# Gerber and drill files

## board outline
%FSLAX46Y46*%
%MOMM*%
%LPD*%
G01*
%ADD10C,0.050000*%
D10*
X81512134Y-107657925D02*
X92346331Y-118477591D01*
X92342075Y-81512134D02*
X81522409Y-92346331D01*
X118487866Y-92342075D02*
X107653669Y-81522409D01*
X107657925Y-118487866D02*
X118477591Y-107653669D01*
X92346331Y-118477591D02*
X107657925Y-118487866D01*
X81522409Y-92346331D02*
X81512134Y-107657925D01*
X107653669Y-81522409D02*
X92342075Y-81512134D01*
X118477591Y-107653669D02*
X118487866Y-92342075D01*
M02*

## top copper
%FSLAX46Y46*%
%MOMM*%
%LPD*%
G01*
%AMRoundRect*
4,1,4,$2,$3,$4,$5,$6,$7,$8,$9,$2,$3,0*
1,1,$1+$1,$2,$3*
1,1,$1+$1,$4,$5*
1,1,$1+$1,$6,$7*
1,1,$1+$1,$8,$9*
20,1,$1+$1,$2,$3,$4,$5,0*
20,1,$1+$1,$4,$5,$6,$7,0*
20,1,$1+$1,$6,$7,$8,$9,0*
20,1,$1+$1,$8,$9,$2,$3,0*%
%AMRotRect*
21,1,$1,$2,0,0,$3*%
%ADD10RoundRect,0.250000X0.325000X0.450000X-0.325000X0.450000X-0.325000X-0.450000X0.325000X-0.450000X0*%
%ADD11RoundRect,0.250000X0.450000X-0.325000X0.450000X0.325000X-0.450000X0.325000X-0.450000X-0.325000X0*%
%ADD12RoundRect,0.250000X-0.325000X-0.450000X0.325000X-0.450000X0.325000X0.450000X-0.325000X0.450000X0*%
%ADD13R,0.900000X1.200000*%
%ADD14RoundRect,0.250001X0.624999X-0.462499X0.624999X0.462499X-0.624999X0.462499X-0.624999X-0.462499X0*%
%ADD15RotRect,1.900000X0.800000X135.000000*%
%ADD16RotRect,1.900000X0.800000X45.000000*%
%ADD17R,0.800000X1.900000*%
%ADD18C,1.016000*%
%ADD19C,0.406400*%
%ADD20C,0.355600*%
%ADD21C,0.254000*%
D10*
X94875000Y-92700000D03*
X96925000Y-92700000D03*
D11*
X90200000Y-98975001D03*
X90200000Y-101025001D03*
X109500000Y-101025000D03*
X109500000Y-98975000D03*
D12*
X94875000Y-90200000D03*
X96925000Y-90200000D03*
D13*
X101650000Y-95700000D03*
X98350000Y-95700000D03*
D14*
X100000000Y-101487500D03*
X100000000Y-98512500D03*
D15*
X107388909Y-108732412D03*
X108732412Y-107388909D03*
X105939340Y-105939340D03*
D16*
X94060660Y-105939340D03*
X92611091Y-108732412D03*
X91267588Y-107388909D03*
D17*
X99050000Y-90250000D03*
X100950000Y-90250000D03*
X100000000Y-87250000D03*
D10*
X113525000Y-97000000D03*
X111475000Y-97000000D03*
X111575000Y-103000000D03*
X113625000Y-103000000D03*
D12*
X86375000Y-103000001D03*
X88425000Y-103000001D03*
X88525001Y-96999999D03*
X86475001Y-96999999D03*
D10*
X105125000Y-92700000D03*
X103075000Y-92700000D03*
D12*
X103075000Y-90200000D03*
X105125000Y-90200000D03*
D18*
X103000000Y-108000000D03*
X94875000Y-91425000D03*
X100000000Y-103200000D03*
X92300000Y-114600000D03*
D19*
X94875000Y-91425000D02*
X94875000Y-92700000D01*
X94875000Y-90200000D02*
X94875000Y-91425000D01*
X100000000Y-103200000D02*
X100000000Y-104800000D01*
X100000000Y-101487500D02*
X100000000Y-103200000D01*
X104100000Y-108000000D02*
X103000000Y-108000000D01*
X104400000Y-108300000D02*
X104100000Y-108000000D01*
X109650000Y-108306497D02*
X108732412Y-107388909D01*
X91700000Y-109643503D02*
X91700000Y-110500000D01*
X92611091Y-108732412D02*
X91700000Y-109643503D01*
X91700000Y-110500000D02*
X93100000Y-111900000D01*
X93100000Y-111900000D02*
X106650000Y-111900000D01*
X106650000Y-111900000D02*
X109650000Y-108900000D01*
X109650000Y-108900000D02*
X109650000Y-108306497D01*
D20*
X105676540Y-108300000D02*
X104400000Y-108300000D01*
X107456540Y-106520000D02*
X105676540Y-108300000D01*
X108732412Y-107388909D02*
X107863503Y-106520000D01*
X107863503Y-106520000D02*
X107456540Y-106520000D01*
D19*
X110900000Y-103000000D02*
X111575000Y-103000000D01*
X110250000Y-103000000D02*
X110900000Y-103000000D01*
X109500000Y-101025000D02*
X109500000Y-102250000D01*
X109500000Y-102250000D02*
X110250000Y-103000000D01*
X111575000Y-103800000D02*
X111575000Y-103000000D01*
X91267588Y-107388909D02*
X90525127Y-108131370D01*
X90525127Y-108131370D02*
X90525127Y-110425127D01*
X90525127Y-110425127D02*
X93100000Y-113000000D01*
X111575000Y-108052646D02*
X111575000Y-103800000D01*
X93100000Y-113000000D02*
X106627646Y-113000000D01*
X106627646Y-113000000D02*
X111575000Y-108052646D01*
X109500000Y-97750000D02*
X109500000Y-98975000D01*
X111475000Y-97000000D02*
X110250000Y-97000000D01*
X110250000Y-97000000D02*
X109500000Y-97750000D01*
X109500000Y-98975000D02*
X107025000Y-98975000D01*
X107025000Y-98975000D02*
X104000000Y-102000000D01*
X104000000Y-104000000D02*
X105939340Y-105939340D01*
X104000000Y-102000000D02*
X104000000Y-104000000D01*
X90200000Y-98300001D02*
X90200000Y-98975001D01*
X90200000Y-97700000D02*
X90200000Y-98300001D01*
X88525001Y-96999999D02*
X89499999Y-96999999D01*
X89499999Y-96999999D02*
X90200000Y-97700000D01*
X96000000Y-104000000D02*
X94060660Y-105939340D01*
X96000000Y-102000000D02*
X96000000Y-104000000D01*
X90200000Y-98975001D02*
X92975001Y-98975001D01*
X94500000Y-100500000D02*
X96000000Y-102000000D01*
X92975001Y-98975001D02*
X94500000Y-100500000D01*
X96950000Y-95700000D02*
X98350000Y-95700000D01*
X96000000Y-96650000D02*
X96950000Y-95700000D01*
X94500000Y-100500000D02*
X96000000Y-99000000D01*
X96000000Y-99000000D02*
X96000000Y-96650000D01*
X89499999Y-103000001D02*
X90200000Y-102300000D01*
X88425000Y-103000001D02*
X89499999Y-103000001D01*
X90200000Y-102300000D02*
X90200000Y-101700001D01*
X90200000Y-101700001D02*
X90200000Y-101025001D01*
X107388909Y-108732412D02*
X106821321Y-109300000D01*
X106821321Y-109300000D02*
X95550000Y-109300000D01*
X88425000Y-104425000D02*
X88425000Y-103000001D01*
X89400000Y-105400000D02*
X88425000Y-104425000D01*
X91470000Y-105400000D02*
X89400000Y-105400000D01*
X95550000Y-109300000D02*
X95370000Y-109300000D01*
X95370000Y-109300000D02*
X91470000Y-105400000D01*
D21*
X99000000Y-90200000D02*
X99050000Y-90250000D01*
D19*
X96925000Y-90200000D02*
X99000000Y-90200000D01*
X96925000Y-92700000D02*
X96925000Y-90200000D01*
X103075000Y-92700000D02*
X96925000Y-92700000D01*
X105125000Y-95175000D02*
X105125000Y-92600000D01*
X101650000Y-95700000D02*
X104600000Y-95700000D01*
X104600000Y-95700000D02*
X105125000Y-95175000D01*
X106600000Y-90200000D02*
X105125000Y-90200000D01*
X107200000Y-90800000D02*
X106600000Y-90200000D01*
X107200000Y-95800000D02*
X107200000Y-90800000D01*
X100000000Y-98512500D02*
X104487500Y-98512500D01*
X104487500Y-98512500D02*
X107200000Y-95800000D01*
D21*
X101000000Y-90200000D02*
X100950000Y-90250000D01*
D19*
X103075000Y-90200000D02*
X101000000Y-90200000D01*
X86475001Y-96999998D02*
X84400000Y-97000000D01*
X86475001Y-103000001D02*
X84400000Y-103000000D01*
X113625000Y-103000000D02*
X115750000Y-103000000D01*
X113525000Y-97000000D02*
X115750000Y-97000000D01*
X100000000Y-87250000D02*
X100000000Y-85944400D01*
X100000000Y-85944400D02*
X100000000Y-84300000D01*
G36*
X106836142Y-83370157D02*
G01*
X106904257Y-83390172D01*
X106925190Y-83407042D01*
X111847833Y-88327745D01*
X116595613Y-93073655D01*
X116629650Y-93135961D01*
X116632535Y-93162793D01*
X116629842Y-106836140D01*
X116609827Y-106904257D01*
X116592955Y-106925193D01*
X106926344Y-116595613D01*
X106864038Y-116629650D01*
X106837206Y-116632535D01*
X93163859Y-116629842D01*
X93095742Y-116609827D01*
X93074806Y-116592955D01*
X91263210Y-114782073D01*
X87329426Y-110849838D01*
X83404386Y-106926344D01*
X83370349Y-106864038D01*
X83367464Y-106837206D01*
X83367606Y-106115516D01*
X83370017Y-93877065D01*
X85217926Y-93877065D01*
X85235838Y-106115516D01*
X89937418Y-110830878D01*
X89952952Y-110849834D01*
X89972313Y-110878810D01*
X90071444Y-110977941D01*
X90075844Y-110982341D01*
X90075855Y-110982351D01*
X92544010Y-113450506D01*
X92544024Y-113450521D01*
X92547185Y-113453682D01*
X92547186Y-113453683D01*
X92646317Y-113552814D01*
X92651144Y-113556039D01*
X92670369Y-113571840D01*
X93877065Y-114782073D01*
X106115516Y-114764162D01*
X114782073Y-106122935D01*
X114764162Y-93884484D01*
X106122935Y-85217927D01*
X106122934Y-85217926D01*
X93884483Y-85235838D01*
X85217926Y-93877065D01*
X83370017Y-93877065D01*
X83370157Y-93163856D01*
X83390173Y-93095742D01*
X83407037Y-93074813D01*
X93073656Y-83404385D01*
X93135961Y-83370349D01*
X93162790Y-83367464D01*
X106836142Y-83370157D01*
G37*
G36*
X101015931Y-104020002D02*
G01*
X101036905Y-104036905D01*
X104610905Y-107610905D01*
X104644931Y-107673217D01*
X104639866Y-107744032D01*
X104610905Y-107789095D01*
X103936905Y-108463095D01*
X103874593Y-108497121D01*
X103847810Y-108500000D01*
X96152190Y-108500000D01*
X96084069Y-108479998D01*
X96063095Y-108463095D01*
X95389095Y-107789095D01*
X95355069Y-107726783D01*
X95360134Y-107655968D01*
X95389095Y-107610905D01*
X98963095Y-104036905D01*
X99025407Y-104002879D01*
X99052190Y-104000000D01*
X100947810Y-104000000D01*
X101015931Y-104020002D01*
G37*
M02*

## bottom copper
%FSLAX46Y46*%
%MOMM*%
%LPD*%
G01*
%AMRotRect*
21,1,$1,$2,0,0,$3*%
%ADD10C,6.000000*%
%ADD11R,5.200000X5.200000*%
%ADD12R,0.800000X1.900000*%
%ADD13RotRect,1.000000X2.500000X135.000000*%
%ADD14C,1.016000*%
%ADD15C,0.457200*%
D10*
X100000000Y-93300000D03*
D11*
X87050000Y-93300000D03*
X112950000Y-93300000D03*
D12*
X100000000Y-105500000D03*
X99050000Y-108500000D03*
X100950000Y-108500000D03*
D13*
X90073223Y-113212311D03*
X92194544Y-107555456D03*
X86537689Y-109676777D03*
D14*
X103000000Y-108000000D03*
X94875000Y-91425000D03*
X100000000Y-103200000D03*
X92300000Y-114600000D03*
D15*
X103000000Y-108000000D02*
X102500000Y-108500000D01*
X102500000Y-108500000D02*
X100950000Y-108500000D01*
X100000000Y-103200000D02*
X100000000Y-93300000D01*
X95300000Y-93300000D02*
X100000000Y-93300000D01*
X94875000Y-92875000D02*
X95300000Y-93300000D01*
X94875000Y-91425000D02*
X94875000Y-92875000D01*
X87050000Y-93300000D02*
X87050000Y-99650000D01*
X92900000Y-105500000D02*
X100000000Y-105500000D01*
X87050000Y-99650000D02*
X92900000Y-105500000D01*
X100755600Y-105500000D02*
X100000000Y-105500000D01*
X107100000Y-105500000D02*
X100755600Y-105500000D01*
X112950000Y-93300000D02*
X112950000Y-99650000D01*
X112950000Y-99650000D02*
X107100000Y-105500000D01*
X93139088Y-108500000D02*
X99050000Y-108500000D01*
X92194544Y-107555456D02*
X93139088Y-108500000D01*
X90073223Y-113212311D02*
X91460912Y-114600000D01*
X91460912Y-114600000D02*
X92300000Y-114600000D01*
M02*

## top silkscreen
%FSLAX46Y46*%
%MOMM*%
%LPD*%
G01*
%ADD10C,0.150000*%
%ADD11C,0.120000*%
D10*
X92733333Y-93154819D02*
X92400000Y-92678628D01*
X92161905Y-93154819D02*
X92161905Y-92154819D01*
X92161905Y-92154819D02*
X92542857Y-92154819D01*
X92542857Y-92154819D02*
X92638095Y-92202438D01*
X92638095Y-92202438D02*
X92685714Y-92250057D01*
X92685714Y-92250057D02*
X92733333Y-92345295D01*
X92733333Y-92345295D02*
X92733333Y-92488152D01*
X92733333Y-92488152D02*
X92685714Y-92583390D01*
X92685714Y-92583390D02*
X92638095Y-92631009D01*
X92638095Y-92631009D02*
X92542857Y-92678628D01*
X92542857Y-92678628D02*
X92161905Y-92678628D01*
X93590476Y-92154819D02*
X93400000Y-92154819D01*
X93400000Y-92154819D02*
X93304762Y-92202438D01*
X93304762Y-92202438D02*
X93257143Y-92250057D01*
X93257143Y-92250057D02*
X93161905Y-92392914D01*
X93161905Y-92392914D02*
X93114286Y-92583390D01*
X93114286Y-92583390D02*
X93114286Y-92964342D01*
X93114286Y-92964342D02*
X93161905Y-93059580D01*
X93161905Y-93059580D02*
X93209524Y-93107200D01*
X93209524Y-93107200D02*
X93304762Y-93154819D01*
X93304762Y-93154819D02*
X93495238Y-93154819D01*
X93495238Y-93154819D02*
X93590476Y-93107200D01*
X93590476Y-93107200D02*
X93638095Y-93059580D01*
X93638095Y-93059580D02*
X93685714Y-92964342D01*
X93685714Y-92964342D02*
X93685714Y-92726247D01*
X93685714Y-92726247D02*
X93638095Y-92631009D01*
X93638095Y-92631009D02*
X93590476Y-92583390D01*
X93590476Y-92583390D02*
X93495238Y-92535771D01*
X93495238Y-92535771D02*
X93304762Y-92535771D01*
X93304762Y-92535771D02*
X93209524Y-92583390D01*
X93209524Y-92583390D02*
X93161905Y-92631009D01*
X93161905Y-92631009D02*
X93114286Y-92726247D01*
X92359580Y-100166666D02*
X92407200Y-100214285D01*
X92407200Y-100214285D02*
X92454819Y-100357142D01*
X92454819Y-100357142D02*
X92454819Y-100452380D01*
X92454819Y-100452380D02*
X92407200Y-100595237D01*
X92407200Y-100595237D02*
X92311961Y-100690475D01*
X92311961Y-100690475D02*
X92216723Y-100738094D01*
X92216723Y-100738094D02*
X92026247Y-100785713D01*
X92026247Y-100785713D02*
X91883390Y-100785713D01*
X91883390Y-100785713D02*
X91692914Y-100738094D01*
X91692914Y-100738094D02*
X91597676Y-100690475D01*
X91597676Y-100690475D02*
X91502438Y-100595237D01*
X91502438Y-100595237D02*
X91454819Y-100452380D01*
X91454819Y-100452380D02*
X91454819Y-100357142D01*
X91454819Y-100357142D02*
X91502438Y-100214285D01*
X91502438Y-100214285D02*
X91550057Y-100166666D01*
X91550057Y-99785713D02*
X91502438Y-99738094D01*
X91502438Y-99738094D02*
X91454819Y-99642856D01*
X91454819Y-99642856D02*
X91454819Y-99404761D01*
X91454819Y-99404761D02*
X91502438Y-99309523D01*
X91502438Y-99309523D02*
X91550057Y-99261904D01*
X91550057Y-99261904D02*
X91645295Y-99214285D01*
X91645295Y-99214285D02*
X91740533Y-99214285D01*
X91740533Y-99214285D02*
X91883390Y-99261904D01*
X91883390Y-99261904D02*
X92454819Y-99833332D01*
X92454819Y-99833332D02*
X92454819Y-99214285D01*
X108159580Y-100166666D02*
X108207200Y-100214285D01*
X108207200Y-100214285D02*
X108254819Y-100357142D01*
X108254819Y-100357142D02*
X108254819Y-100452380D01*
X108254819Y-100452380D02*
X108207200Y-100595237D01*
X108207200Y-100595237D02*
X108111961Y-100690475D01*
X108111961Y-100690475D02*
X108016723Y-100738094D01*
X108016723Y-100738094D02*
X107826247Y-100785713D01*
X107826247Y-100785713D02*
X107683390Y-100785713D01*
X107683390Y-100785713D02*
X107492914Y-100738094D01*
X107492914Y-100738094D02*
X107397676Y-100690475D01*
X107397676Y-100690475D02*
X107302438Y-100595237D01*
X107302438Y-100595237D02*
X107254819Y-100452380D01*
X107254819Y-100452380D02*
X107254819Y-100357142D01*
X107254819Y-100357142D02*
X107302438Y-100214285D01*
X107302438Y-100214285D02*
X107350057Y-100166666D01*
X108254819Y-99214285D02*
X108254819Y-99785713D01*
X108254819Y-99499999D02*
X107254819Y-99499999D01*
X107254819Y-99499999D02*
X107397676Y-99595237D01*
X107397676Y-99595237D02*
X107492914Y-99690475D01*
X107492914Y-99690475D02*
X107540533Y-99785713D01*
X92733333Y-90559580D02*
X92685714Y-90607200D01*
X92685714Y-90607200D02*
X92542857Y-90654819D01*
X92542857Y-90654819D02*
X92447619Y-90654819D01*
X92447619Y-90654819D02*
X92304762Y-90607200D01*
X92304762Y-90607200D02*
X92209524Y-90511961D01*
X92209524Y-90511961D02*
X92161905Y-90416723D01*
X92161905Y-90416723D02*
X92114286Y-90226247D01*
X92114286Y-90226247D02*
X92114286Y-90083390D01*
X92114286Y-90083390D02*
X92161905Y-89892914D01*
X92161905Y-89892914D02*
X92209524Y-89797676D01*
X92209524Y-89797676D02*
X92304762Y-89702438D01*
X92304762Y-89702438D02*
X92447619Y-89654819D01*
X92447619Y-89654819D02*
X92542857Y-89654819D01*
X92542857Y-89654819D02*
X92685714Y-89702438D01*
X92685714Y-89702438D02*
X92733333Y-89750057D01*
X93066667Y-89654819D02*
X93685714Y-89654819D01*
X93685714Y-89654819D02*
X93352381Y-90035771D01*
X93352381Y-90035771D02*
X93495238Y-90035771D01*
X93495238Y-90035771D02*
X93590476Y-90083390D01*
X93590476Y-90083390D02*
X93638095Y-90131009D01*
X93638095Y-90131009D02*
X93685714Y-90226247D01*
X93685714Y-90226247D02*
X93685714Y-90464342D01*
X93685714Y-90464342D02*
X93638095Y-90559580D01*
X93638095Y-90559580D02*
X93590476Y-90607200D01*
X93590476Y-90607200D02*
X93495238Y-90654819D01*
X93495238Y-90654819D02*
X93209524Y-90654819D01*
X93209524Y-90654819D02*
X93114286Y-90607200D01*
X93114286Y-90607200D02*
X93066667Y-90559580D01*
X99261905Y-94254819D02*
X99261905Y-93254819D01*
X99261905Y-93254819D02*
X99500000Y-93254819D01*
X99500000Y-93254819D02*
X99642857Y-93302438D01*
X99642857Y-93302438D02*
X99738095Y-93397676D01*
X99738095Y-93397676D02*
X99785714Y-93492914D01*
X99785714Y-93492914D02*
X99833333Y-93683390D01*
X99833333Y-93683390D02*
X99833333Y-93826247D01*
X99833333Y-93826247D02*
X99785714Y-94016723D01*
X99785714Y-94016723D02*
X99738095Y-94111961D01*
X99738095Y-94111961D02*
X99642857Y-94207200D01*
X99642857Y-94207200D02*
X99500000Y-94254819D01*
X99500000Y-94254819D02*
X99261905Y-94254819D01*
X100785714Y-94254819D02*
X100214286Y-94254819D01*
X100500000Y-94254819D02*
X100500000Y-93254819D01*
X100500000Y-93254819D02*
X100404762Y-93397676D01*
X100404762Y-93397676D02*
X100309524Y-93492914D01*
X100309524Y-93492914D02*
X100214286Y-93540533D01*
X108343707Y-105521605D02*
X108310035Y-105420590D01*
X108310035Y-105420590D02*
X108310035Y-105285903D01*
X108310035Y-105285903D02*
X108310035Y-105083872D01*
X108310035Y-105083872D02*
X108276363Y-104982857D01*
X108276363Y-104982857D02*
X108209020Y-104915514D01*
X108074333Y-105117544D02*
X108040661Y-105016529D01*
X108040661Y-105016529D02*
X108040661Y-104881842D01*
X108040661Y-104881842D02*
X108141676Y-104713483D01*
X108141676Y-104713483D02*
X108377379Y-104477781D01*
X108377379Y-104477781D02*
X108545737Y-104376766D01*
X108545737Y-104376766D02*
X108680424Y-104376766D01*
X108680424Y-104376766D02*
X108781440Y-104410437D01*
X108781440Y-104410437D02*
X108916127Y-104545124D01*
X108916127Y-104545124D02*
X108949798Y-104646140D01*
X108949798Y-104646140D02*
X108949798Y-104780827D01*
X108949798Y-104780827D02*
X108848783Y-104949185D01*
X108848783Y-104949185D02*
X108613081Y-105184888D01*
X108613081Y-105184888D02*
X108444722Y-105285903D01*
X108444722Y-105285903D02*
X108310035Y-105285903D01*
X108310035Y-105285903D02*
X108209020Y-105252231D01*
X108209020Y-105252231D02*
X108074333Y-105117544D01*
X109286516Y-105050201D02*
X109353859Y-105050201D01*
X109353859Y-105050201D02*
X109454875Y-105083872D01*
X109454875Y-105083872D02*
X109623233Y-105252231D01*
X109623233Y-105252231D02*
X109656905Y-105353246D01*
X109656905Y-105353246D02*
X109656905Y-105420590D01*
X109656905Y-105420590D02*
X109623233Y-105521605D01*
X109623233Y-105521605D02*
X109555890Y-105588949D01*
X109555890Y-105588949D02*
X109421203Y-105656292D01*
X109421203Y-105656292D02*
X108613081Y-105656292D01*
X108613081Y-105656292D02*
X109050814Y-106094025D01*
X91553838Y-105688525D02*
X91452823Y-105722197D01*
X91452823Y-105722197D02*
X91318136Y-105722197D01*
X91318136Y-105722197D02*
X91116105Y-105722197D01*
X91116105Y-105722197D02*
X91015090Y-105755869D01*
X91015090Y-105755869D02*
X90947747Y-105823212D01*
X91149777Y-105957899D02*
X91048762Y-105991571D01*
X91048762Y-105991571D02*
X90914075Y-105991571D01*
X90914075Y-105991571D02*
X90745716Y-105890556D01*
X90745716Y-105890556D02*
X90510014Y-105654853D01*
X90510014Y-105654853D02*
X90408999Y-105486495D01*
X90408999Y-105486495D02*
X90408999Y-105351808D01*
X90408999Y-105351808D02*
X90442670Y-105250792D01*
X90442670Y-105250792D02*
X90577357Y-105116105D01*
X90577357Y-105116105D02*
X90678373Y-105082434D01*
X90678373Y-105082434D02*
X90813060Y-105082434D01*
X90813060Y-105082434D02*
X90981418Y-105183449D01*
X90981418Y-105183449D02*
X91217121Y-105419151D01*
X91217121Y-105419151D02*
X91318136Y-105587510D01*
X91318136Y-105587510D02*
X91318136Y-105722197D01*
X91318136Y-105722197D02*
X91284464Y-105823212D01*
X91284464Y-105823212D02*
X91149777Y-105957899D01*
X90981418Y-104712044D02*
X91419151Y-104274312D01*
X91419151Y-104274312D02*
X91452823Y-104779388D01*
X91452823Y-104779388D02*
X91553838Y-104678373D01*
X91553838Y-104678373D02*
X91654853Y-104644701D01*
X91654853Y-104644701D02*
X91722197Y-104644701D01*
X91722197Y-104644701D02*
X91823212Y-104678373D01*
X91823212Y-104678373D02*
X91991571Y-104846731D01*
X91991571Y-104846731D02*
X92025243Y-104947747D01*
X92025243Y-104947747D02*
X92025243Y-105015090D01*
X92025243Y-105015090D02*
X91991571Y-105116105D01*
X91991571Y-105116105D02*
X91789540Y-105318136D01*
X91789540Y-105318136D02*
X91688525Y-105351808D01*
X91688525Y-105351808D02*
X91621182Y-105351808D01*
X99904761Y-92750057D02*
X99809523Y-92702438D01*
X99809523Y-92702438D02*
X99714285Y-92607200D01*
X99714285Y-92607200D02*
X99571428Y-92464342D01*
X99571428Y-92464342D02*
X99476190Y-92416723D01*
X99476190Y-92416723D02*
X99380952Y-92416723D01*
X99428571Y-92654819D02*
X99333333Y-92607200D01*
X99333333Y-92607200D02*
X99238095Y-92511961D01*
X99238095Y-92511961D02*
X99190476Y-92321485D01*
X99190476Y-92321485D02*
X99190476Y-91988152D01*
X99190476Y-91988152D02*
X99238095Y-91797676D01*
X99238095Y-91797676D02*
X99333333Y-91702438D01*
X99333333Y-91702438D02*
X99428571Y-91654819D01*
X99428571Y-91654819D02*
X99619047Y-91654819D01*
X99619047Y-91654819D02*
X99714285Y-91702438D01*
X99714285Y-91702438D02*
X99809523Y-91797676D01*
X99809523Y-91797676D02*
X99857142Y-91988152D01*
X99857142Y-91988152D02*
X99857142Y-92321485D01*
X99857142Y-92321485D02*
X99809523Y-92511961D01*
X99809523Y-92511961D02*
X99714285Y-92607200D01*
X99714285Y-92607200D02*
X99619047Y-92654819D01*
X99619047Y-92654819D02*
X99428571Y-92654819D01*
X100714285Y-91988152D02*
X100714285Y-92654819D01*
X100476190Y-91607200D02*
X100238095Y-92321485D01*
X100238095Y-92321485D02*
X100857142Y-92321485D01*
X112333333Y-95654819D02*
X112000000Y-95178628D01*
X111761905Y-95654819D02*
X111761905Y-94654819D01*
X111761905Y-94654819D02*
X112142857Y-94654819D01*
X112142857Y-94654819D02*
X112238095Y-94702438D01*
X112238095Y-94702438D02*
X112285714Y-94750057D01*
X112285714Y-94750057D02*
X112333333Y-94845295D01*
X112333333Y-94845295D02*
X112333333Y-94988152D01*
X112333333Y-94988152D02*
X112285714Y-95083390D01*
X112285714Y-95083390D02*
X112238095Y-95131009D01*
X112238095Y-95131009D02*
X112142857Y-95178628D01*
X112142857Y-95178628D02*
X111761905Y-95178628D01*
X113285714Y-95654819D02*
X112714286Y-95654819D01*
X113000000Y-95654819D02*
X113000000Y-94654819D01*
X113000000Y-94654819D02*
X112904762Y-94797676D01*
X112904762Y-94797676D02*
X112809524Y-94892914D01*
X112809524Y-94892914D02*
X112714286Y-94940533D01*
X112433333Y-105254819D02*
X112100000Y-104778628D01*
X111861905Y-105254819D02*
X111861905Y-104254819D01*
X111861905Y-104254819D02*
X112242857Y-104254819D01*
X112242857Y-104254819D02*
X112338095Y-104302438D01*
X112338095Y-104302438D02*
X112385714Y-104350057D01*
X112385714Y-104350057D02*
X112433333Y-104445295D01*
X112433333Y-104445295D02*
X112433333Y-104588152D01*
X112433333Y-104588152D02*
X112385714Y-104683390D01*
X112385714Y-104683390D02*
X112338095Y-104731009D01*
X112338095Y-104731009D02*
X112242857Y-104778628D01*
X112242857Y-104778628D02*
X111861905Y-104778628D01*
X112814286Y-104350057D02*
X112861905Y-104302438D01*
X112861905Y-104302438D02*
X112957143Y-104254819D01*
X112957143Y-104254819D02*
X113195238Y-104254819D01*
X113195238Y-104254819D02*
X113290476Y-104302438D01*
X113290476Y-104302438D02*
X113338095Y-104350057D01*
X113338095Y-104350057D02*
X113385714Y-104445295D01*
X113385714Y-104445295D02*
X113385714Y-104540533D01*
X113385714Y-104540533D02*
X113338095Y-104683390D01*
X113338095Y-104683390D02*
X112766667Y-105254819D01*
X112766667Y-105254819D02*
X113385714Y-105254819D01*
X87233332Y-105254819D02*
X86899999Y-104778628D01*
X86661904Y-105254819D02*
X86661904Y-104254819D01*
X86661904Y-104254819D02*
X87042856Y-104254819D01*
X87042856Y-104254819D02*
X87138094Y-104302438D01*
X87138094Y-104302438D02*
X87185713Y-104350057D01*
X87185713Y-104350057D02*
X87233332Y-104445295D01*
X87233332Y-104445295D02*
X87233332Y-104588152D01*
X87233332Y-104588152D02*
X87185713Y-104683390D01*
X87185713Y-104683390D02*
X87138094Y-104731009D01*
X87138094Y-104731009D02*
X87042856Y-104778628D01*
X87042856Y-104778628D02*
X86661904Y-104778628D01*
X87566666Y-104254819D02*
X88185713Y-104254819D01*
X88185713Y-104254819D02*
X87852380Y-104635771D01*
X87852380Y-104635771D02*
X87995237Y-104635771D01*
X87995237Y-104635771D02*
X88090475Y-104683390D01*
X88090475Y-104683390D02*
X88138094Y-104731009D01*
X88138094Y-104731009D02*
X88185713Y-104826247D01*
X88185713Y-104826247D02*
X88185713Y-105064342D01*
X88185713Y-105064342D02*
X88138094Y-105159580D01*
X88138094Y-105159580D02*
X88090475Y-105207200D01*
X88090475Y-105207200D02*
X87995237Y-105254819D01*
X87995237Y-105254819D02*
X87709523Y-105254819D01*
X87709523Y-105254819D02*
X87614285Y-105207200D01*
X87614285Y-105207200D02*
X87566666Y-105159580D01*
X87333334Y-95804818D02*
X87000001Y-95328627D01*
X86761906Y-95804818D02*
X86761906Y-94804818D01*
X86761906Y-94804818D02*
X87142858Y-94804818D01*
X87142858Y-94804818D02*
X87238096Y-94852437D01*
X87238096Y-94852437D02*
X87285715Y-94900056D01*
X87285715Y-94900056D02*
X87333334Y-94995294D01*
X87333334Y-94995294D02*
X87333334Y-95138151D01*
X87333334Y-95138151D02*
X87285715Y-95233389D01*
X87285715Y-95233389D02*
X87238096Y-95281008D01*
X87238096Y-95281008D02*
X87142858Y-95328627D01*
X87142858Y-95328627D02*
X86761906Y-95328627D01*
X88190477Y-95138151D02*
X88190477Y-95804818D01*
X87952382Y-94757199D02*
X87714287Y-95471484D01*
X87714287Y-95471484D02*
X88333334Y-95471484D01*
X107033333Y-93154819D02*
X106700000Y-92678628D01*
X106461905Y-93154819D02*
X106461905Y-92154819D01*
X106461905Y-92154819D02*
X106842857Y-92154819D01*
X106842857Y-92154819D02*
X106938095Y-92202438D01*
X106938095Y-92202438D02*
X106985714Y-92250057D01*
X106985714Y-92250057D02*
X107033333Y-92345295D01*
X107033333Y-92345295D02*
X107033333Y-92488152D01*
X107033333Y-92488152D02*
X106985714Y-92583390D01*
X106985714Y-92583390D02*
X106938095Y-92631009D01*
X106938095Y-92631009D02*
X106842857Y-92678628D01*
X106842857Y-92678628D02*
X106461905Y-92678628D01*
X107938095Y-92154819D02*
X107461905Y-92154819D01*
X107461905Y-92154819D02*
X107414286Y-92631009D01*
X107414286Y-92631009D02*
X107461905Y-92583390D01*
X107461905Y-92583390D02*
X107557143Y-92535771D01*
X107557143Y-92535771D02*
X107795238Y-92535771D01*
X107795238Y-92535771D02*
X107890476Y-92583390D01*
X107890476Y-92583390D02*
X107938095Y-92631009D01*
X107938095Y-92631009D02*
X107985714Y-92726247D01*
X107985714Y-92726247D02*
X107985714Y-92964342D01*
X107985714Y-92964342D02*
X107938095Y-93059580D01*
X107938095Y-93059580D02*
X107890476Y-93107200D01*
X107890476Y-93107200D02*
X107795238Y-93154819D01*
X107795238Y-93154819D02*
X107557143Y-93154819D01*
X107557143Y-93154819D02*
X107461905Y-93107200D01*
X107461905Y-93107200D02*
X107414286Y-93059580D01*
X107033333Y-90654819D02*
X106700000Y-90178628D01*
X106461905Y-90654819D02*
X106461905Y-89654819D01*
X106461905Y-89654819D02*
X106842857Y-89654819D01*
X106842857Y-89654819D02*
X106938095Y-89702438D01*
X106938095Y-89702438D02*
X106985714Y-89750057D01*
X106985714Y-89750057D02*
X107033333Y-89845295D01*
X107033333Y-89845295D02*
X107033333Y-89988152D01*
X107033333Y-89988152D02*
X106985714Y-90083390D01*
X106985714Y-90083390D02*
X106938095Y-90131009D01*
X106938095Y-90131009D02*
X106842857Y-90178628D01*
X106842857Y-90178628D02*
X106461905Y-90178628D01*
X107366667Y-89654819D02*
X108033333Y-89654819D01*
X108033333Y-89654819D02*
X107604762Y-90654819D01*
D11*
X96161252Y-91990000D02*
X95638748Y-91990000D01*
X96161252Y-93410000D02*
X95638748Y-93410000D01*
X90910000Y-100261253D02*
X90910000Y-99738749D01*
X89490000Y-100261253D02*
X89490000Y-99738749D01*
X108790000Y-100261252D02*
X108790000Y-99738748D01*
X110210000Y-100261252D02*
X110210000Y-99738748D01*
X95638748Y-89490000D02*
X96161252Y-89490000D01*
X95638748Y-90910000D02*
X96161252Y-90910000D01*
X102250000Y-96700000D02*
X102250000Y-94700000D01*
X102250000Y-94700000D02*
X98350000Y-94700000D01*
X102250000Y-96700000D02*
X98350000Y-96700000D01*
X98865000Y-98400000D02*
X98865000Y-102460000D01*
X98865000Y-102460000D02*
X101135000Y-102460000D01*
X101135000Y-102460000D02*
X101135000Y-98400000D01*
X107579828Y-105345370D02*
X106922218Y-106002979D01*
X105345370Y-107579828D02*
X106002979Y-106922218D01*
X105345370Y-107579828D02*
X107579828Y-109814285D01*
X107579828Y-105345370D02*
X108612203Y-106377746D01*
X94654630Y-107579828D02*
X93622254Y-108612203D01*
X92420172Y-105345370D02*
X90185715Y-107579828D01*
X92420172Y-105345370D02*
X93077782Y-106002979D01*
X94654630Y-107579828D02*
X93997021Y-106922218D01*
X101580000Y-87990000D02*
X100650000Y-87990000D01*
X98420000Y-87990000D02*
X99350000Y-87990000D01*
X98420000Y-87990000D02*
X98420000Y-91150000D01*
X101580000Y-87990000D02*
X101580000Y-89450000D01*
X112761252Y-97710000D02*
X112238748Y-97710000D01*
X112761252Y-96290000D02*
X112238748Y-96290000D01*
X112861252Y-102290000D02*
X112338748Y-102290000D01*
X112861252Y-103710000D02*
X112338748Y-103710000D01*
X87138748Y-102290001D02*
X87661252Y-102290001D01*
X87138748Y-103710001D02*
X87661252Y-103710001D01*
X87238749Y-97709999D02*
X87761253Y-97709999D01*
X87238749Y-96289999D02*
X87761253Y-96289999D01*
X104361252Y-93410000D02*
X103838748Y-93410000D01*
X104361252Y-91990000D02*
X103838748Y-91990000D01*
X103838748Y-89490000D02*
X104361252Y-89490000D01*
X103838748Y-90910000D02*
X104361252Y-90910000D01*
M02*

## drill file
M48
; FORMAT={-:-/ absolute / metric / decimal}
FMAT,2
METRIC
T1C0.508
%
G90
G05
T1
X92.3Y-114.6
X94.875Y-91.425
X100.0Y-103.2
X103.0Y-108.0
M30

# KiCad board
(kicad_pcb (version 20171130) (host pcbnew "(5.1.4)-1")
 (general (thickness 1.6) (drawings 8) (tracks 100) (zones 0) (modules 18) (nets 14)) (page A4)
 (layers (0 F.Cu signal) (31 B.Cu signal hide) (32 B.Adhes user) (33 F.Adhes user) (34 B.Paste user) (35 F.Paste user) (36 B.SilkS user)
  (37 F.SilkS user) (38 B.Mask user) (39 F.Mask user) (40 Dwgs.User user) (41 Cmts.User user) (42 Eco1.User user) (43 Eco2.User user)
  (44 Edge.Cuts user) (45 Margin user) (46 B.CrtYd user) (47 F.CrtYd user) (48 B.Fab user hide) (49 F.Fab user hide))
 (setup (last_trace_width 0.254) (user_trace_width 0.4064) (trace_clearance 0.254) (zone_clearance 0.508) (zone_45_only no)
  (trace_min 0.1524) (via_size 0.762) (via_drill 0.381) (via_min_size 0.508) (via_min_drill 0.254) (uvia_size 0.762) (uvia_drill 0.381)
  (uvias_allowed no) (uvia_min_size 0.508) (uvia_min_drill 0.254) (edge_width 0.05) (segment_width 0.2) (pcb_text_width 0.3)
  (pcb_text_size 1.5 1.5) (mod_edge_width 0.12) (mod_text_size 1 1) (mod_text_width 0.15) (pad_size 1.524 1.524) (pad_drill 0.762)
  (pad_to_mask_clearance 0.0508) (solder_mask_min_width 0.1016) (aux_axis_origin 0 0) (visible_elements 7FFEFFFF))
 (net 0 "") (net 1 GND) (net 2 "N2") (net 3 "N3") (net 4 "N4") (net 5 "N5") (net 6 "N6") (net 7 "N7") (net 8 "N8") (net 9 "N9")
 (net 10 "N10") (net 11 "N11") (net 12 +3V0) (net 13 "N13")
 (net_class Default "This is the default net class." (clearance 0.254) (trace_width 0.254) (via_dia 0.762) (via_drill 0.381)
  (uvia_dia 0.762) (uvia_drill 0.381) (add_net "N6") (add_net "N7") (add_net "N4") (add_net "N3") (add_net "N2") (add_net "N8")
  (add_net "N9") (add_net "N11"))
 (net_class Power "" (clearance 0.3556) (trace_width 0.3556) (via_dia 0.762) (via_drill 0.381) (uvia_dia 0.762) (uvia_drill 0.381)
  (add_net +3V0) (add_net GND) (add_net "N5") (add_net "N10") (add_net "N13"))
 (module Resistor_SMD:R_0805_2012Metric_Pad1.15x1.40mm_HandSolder (layer F.Cu) (at 95.9 92.7 180)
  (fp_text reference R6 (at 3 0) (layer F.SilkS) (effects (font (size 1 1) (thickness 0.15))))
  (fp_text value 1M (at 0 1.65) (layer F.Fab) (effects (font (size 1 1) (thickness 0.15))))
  (fp_line (start -0.261252 0.71) (end 0.261252 0.71) (layer F.SilkS) (width 0.12))
  (fp_line (start -0.261252 -0.71) (end 0.261252 -0.71) (layer F.SilkS) (width 0.12))
  (pad 2 smd roundrect (at 1.025 0 180) (size 1.15 1.4) (layers F.Cu F.Paste F.Mask) (roundrect_rratio 0.217391) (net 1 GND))
  (pad 1 smd roundrect (at -1.025 0 180) (size 1.15 1.4) (layers F.Cu F.Paste F.Mask) (roundrect_rratio 0.217391) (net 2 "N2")))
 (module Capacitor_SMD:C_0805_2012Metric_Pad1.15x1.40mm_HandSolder (layer F.Cu) (at 90.2 100.000001 90)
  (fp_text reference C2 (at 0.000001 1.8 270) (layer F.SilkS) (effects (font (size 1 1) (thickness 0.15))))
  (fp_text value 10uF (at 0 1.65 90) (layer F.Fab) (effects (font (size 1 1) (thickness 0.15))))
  (fp_line (start -0.261252 0.71) (end 0.261252 0.71) (layer F.SilkS) (width 0.12))
  (fp_line (start -0.261252 -0.71) (end 0.261252 -0.71) (layer F.SilkS) (width 0.12))
  (pad 2 smd roundrect (at 1.025 0 90) (size 1.15 1.4) (layers F.Cu F.Paste F.Mask) (roundrect_rratio 0.217391) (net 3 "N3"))
  (pad 1 smd roundrect (at -1.025 0 90) (size 1.15 1.4) (layers F.Cu F.Paste F.Mask) (roundrect_rratio 0.217391) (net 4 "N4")))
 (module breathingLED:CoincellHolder (layer B.Cu) (at 100 93.3) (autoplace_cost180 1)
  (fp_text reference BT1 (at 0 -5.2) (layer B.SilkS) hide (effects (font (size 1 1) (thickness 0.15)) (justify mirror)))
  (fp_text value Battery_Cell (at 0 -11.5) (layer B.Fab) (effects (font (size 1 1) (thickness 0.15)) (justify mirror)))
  (pad 2 smd circle (at 0 0) (size 6 6) (layers B.Cu B.Paste B.Mask) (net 1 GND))
  (pad 1 smd rect (at -12.95 0) (size 5.2 5.2) (layers B.Cu B.Paste B.Mask) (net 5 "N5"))
  (pad 1 smd rect (at 12.95 0) (size 5.2 5.2) (layers B.Cu B.Paste B.Mask) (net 5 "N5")))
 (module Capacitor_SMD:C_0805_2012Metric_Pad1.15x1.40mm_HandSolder (layer F.Cu) (at 109.5 100 90)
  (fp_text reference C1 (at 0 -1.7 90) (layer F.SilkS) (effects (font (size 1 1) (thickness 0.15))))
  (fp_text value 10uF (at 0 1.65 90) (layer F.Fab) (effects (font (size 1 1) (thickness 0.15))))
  (fp_line (start -0.261252 -0.71) (end 0.261252 -0.71) (layer F.SilkS) (width 0.12))
  (fp_line (start -0.261252 0.71) (end 0.261252 0.71) (layer F.SilkS) (width 0.12))
  (pad 1 smd roundrect (at -1.025 0 90) (size 1.15 1.4) (layers F.Cu F.Paste F.Mask) (roundrect_rratio 0.217391) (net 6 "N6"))
  (pad 2 smd roundrect (at 1.025 0 90) (size 1.15 1.4) (layers F.Cu F.Paste F.Mask) (roundrect_rratio 0.217391) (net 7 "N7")))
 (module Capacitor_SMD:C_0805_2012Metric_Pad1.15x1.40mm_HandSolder (layer F.Cu) (at 95.9 90.2)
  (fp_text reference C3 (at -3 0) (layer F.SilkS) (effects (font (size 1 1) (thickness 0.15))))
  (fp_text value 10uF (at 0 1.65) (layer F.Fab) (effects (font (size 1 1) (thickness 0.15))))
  (fp_line (start -0.261252 -0.71) (end 0.261252 -0.71) (layer F.SilkS) (width 0.12))
  (fp_line (start -0.261252 0.71) (end 0.261252 0.71) (layer F.SilkS) (width 0.12))
  (pad 1 smd roundrect (at -1.025 0) (size 1.15 1.4) (layers F.Cu F.Paste F.Mask) (roundrect_rratio 0.217391) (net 1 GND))
  (pad 2 smd roundrect (at 1.025 0) (size 1.15 1.4) (layers F.Cu F.Paste F.Mask) (roundrect_rratio 0.217391) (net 2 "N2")))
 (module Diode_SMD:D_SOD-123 (layer F.Cu) (at 100 95.7 180)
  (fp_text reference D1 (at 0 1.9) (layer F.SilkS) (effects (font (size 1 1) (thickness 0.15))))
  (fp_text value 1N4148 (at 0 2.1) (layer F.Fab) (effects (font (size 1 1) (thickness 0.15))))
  (fp_line (start -2.25 -1) (end -2.25 1) (layer F.SilkS) (width 0.12))
  (fp_line (start -2.25 1) (end 1.65 1) (layer F.SilkS) (width 0.12))
  (fp_line (start -2.25 -1) (end 1.65 -1) (layer F.SilkS) (width 0.12))
  (pad 1 smd rect (at -1.65 0 180) (size 0.9 1.2) (layers F.Cu F.Paste F.Mask) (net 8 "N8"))
  (pad 2 smd rect (at 1.65 0 180) (size 0.9 1.2) (layers F.Cu F.Paste F.Mask) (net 3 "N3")))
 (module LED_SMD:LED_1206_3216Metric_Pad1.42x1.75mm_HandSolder (layer F.Cu) (at 100 100 90)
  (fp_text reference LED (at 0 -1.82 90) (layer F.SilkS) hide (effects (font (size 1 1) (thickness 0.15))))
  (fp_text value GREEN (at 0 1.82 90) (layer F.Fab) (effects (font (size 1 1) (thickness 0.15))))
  (fp_line (start 1.6 -1.135) (end -2.46 -1.135) (layer F.SilkS) (width 0.12))
  (fp_line (start -2.46 -1.135) (end -2.46 1.135) (layer F.SilkS) (width 0.12))
  (fp_line (start -2.46 1.135) (end 1.6 1.135) (layer F.SilkS) (width 0.12))
  (pad 1 smd roundrect (at -1.4875 0 90) (size 1.425 1.75) (layers F.Cu F.Paste F.Mask) (roundrect_rratio 0.175439) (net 1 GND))
  (pad 2 smd roundrect (at 1.4875 0 90) (size 1.425 1.75) (layers F.Cu F.Paste F.Mask) (roundrect_rratio 0.175439) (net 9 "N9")))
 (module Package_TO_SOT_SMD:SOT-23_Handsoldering (layer B.Cu) (at 100 107 90)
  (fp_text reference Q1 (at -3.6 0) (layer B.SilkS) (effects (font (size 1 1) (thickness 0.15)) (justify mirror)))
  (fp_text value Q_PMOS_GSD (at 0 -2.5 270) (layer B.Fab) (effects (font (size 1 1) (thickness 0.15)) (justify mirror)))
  (pad 3 smd rect (at 1.5 0 90) (size 1.9 0.8) (layers B.Cu B.Paste B.Mask) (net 5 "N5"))
  (pad 2 smd rect (at -1.5 -0.95 90) (size 1.9 0.8) (layers B.Cu B.Paste B.Mask) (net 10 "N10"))
  (pad 1 smd rect (at -1.5 0.95 90) (size 1.9 0.8) (layers B.Cu B.Paste B.Mask) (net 1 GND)))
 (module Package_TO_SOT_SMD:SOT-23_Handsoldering (layer F.Cu) (at 107 107 135)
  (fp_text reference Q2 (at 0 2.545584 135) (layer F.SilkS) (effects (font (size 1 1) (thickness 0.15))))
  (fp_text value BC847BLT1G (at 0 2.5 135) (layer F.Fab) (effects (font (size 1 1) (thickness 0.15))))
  (fp_line (start 0.76 1.58) (end 0.76 0.65) (layer F.SilkS) (width 0.12))
  (fp_line (start 0.76 -1.58) (end 0.76 -0.65) (layer F.SilkS) (width 0.12))
  (fp_line (start 0.76 -1.58) (end -2.4 -1.58) (layer F.SilkS) (width 0.12))
  (fp_line (start 0.76 1.58) (end -0.7 1.58) (layer F.SilkS) (width 0.12))
  (pad 1 smd rect (at -1.5 -0.95 135) (size 1.9 0.8) (layers F.Cu F.Paste F.Mask) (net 4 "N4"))
  (pad 2 smd rect (at -1.5 0.95 135) (size 1.9 0.8) (layers F.Cu F.Paste F.Mask) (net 1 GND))
  (pad 3 smd rect (at 1.5 0 135) (size 1.9 0.8) (layers F.Cu F.Paste F.Mask) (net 7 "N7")))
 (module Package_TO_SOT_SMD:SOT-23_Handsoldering (layer F.Cu) (at 93 107 45)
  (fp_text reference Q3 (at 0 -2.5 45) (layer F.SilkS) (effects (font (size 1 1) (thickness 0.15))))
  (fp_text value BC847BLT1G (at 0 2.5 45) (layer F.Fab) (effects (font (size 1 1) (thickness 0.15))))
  (fp_line (start 0.76 1.58) (end -0.7 1.58) (layer F.SilkS) (width 0.12))
  (fp_line (start 0.76 -1.58) (end -2.4 -1.58) (layer F.SilkS) (width 0.12))
  (fp_line (start 0.76 -1.58) (end 0.76 -0.65) (layer F.SilkS) (width 0.12))
  (fp_line (start 0.76 1.58) (end 0.76 0.65) (layer F.SilkS) (width 0.12))
  (pad 3 smd rect (at 1.5 0 45) (size 1.9 0.8) (layers F.Cu F.Paste F.Mask) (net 3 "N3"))
  (pad 2 smd rect (at -1.5 0.95 45) (size 1.9 0.8) (layers F.Cu F.Paste F.Mask) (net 1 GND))
  (pad 1 smd rect (at -1.5 -0.95 45) (size 1.9 0.8) (layers F.Cu F.Paste F.Mask) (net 6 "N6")))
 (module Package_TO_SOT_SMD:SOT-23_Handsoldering (layer F.Cu) (at 100 88.75 90)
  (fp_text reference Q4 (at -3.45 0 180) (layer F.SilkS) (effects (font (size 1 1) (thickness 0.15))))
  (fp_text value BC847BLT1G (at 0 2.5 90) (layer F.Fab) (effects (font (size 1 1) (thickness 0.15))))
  (fp_line (start 0.76 1.58) (end 0.76 0.65) (layer F.SilkS) (width 0.12))
  (fp_line (start 0.76 -1.58) (end 0.76 -0.65) (layer F.SilkS) (width 0.12))
  (fp_line (start 0.76 -1.58) (end -2.4 -1.58) (layer F.SilkS) (width 0.12))
  (fp_line (start 0.76 1.58) (end -0.7 1.58) (layer F.SilkS) (width 0.12))
  (pad 1 smd rect (at -1.5 -0.95 90) (size 1.9 0.8) (layers F.Cu F.Paste F.Mask) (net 2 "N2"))
  (pad 2 smd rect (at -1.5 0.95 90) (size 1.9 0.8) (layers F.Cu F.Paste F.Mask) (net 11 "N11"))
  (pad 3 smd rect (at 1.5 0 90) (size 1.9 0.8) (layers F.Cu F.Paste F.Mask) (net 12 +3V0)))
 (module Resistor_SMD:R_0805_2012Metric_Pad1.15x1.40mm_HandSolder (layer F.Cu) (at 112.5 97 180)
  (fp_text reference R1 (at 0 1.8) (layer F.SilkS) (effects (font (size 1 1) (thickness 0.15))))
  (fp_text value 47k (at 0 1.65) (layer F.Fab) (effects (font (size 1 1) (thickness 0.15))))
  (fp_line (start -0.261252 -0.71) (end 0.261252 -0.71) (layer F.SilkS) (width 0.12))
  (fp_line (start -0.261252 0.71) (end 0.261252 0.71) (layer F.SilkS) (width 0.12))
  (pad 1 smd roundrect (at -1.025 0 180) (size 1.15 1.4) (layers F.Cu F.Paste F.Mask) (roundrect_rratio 0.217391) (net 12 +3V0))
  (pad 2 smd roundrect (at 1.025 0 180) (size 1.15 1.4) (layers F.Cu F.Paste F.Mask) (roundrect_rratio 0.217391) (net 7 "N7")))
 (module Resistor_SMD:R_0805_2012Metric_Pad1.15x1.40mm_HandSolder (layer F.Cu) (at 112.6 103 180)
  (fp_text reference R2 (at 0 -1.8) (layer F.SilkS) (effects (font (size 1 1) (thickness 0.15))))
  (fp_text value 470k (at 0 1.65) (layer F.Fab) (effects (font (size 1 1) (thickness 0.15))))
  (fp_line (start -0.261252 0.71) (end 0.261252 0.71) (layer F.SilkS) (width 0.12))
  (fp_line (start -0.261252 -0.71) (end 0.261252 -0.71) (layer F.SilkS) (width 0.12))
  (pad 2 smd roundrect (at 1.025 0 180) (size 1.15 1.4) (layers F.Cu F.Paste F.Mask) (roundrect_rratio 0.217391) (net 6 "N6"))
  (pad 1 smd roundrect (at -1.025 0 180) (size 1.15 1.4) (layers F.Cu F.Paste F.Mask) (roundrect_rratio 0.217391) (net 12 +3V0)))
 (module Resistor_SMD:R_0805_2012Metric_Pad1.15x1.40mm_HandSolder (layer F.Cu) (at 87.4 103.000001)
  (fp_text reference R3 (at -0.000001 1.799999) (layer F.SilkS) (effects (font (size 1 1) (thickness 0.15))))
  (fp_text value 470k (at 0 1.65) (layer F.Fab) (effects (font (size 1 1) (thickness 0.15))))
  (fp_line (start -0.261252 -0.71) (end 0.261252 -0.71) (layer F.SilkS) (width 0.12))
  (fp_line (start -0.261252 0.71) (end 0.261252 0.71) (layer F.SilkS) (width 0.12))
  (pad 1 smd roundrect (at -1.025 0) (size 1.15 1.4) (layers F.Cu F.Paste F.Mask) (roundrect_rratio 0.217391) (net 12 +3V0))
  (pad 2 smd roundrect (at 1.025 0) (size 1.15 1.4) (layers F.Cu F.Paste F.Mask) (roundrect_rratio 0.217391) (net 4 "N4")))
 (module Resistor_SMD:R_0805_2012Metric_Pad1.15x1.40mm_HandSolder (layer F.Cu) (at 87.500001 96.999999)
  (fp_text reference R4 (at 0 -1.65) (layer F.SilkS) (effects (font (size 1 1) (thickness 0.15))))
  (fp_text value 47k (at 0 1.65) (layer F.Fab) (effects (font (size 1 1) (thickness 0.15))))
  (fp_line (start -0.261252 0.71) (end 0.261252 0.71) (layer F.SilkS) (width 0.12))
  (fp_line (start -0.261252 -0.71) (end 0.261252 -0.71) (layer F.SilkS) (width 0.12))
  (pad 2 smd roundrect (at 1.025 0) (size 1.15 1.4) (layers F.Cu F.Paste F.Mask) (roundrect_rratio 0.217391) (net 3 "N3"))
  (pad 1 smd roundrect (at -1.025 0) (size 1.15 1.4) (layers F.Cu F.Paste F.Mask) (roundrect_rratio 0.217391) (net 12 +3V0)))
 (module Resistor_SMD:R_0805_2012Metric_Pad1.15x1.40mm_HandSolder (layer F.Cu) (at 104.1 92.7 180)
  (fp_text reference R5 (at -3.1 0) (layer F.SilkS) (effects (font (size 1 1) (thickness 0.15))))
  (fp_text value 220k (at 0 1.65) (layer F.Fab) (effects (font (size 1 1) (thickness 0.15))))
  (fp_line (start -0.261252 -0.71) (end 0.261252 -0.71) (layer F.SilkS) (width 0.12))
  (fp_line (start -0.261252 0.71) (end 0.261252 0.71) (layer F.SilkS) (width 0.12))
  (pad 1 smd roundrect (at -1.025 0 180) (size 1.15 1.4) (layers F.Cu F.Paste F.Mask) (roundrect_rratio 0.217391) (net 8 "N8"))
  (pad 2 smd roundrect (at 1.025 0 180) (size 1.15 1.4) (layers F.Cu F.Paste F.Mask) (roundrect_rratio 0.217391) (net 2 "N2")))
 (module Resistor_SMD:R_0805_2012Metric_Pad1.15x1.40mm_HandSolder (layer F.Cu) (at 104.1 90.2)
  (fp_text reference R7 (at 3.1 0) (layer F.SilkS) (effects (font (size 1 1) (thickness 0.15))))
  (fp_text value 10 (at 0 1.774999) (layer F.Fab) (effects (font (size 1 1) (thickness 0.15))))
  (fp_line (start -0.261252 -0.71) (end 0.261252 -0.71) (layer F.SilkS) (width 0.12))
  (fp_line (start -0.261252 0.71) (end 0.261252 0.71) (layer F.SilkS) (width 0.12))
  (pad 1 smd roundrect (at -1.025 0) (size 1.15 1.4) (layers F.Cu F.Paste F.Mask) (roundrect_rratio 0.217391) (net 11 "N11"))
  (pad 2 smd roundrect (at 1.025 0) (size 1.15 1.4) (layers F.Cu F.Paste F.Mask) (roundrect_rratio 0.217391) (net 9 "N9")))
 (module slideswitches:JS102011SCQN (layer B.Cu) (at 90.25 109.5 135)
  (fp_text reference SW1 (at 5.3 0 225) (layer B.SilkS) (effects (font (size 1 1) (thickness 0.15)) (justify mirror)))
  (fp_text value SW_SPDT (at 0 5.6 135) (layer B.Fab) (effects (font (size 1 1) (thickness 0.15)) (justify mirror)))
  (pad 1 smd rect (at -2.5 -2.75 135) (size 1 2.5) (layers B.Cu B.Paste B.Mask) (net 12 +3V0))
  (pad 2 smd rect (at 0 2.75 135) (size 1 2.5) (layers B.Cu B.Paste B.Mask) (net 10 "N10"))
  (pad 3 smd rect (at 2.5 -2.75 135) (size 1 2.5) (layers B.Cu B.Paste B.Mask) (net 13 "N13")))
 (gr_line (start 81.512134 107.657925) (end 92.346331 118.477591) (layer Edge.Cuts) (width 0.05))
 (gr_line (start 92.342075 81.512134) (end 81.522409 92.346331) (layer Edge.Cuts) (width 0.05))
 (gr_line (start 118.487866 92.342075) (end 107.653669 81.522409) (layer Edge.Cuts) (width 0.05))
 (gr_line (start 107.657925 118.487866) (end 118.477591 107.653669) (layer Edge.Cuts) (width 0.05))
 (gr_line (start 92.346331 118.477591) (end 107.657925 118.487866) (layer Edge.Cuts) (width 0.05))
 (gr_line (start 81.522409 92.346331) (end 81.512134 107.657925) (layer Edge.Cuts) (width 0.05))
 (gr_line (start 107.653669 81.522409) (end 92.342075 81.512134) (layer Edge.Cuts) (width 0.05))
 (gr_line (start 118.477591 107.653669) (end 118.487866 92.342075) (layer Edge.Cuts) (width 0.05))
 (via (at 103 108) (size 1.016) (drill 0.508) (layers F.Cu B.Cu) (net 1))
 (segment (start 103 108) (end 102.5 108.5) (width 0.4572) (layer B.Cu) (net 1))
 (segment (start 102.5 108.5) (end 100.95 108.5) (width 0.4572) (layer B.Cu) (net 1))
 (via (at 94.875 91.425) (size 1.016) (drill 0.508) (layers F.Cu B.Cu) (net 1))
 (segment (start 94.875 91.425) (end 94.875 92.7) (width 0.4064) (layer F.Cu) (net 1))
 (segment (start 94.875 90.2) (end 94.875 91.425) (width 0.4064) (layer F.Cu) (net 1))
 (via (at 100 103.2) (size 1.016) (drill 0.508) (layers F.Cu B.Cu) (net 1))
 (segment (start 100 103.2) (end 100 104.8) (width 0.4064) (layer F.Cu) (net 1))
 (segment (start 100 101.4875) (end 100 103.2) (width 0.4064) (layer F.Cu) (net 1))
 (segment (start 100 103.2) (end 100 93.3) (width 0.4572) (layer B.Cu) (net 1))
 (segment (start 104.1 108) (end 103 108) (width 0.4064) (layer F.Cu) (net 1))
 (segment (start 104.4 108.3) (end 104.1 108) (width 0.4064) (layer F.Cu) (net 1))
 (segment (start 95.3 93.3) (end 100 93.3) (width 0.4572) (layer B.Cu) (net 1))
 (segment (start 94.875 92.875) (end 95.3 93.3) (width 0.4572) (layer B.Cu) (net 1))
 (segment (start 94.875 91.425) (end 94.875 92.875) (width 0.4572) (layer B.Cu) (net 1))
 (segment (start 109.65 108.306497) (end 108.732412 107.388909) (width 0.4064) (layer F.Cu) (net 1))
 (segment (start 91.7 109.643503) (end 91.7 110.5) (width 0.4064) (layer F.Cu) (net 1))
 (segment (start 92.611091 108.732412) (end 91.7 109.643503) (width 0.4064) (layer F.Cu) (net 1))
 (segment (start 91.7 110.5) (end 93.1 111.9) (width 0.4064) (layer F.Cu) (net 1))
 (segment (start 93.1 111.9) (end 106.65 111.9) (width 0.4064) (layer F.Cu) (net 1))
 (segment (start 106.65 111.9) (end 109.65 108.9) (width 0.4064) (layer F.Cu) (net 1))
 (segment (start 109.65 108.9) (end 109.65 108.306497) (width 0.4064) (layer F.Cu) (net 1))
 (segment (start 105.67654 108.3) (end 104.4 108.3) (width 0.3556) (layer F.Cu) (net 1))
 (segment (start 107.45654 106.52) (end 105.67654 108.3) (width 0.3556) (layer F.Cu) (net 1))
 (segment (start 108.732412 107.388909) (end 107.863503 106.52) (width 0.3556) (layer F.Cu) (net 1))
 (segment (start 107.863503 106.52) (end 107.45654 106.52) (width 0.3556) (layer F.Cu) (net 1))
 (segment (start 87.05 93.3) (end 87.05 99.65) (width 0.4572) (layer B.Cu) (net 5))
 (segment (start 92.9 105.5) (end 100 105.5) (width 0.4572) (layer B.Cu) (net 5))
 (segment (start 87.05 99.65) (end 92.9 105.5) (width 0.4572) (layer B.Cu) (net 5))
 (segment (start 100.7556 105.5) (end 100 105.5) (width 0.4572) (layer B.Cu) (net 5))
 (segment (start 107.1 105.5) (end 100.7556 105.5) (width 0.4572) (layer B.Cu) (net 5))
 (segment (start 112.95 93.3) (end 112.95 99.65) (width 0.4572) (layer B.Cu) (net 5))
 (segment (start 112.95 99.65) (end 107.1 105.5) (width 0.4572) (layer B.Cu) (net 5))
 (segment (start 110.9 103) (end 111.575 103) (width 0.4064) (layer F.Cu) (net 6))
 (segment (start 110.25 103) (end 110.9 103) (width 0.4064) (layer F.Cu) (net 6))
 (segment (start 109.5 101.025) (end 109.5 102.25) (width 0.4064) (layer F.Cu) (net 6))
 (segment (start 109.5 102.25) (end 110.25 103) (width 0.4064) (layer F.Cu) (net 6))
 (segment (start 111.575 103.8) (end 111.575 103) (width 0.4064) (layer F.Cu) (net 6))
 (segment (start 91.267588 107.388909) (end 90.525127 108.13137) (width 0.4064) (layer F.Cu) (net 6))
 (segment (start 90.525127 108.13137) (end 90.525127 110.425127) (width 0.4064) (layer F.Cu) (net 6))
 (segment (start 90.525127 110.425127) (end 93.1 113) (width 0.4064) (layer F.Cu) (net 6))
 (segment (start 111.575 108.052646) (end 111.575 103.8) (width 0.4064) (layer F.Cu) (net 6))
 (segment (start 93.1 113) (end 106.627646 113) (width 0.4064) (layer F.Cu) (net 6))
 (segment (start 106.627646 113) (end 111.575 108.052646) (width 0.4064) (layer F.Cu) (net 6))
 (segment (start 109.5 97.75) (end 109.5 98.975) (width 0.4064) (layer F.Cu) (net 7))
 (segment (start 111.475 97) (end 110.25 97) (width 0.4064) (layer F.Cu) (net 7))
 (segment (start 110.25 97) (end 109.5 97.75) (width 0.4064) (layer F.Cu) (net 7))
 (segment (start 109.5 98.975) (end 107.025 98.975) (width 0.4064) (layer F.Cu) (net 7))
 (segment (start 107.025 98.975) (end 104 102) (width 0.4064) (layer F.Cu) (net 7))
 (segment (start 104 104) (end 105.93934 105.93934) (width 0.4064) (layer F.Cu) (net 7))
 (segment (start 104 102) (end 104 104) (width 0.4064) (layer F.Cu) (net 7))
 (segment (start 90.2 98.300001) (end 90.2 98.975001) (width 0.4064) (layer F.Cu) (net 3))
 (segment (start 90.2 97.7) (end 90.2 98.300001) (width 0.4064) (layer F.Cu) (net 3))
 (segment (start 88.525001 96.999999) (end 89.499999 96.999999) (width 0.4064) (layer F.Cu) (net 3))
 (segment (start 89.499999 96.999999) (end 90.2 97.7) (width 0.4064) (layer F.Cu) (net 3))
 (segment (start 96 104) (end 94.06066 105.93934) (width 0.4064) (layer F.Cu) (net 3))
 (segment (start 96 102) (end 96 104) (width 0.4064) (layer F.Cu) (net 3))
 (segment (start 90.2 98.975001) (end 92.975001 98.975001) (width 0.4064) (layer F.Cu) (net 3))
 (segment (start 94.5 100.5) (end 96 102) (width 0.4064) (layer F.Cu) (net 3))
 (segment (start 92.975001 98.975001) (end 94.5 100.5) (width 0.4064) (layer F.Cu) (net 3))
 (segment (start 96.95 95.7) (end 98.35 95.7) (width 0.4064) (layer F.Cu) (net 3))
 (segment (start 96 96.65) (end 96.95 95.7) (width 0.4064) (layer F.Cu) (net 3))
 (segment (start 94.5 100.5) (end 96 99) (width 0.4064) (layer F.Cu) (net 3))
 (segment (start 96 99) (end 96 96.65) (width 0.4064) (layer F.Cu) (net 3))
 (segment (start 89.499999 103.000001) (end 90.2 102.3) (width 0.4064) (layer F.Cu) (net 4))
 (segment (start 88.425 103.000001) (end 89.499999 103.000001) (width 0.4064) (layer F.Cu) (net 4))
 (segment (start 90.2 102.3) (end 90.2 101.700001) (width 0.4064) (layer F.Cu) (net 4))
 (segment (start 90.2 101.700001) (end 90.2 101.025001) (width 0.4064) (layer F.Cu) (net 4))
 (segment (start 107.388909 108.732412) (end 106.821321 109.3) (width 0.4064) (layer F.Cu) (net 4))
 (segment (start 106.821321 109.3) (end 95.55 109.3) (width 0.4064) (layer F.Cu) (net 4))
 (segment (start 88.425 104.425) (end 88.425 103.000001) (width 0.4064) (layer F.Cu) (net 4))
 (segment (start 89.4 105.4) (end 88.425 104.425) (width 0.4064) (layer F.Cu) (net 4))
 (segment (start 91.47 105.4) (end 89.4 105.4) (width 0.4064) (layer F.Cu) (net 4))
 (segment (start 95.55 109.3) (end 95.37 109.3) (width 0.4064) (layer F.Cu) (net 4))
 (segment (start 95.37 109.3) (end 91.47 105.4) (width 0.4064) (layer F.Cu) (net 4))
 (segment (start 99 90.2) (end 99.05 90.25) (width 0.254) (layer F.Cu) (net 2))
 (segment (start 96.925 90.2) (end 99 90.2) (width 0.4064) (layer F.Cu) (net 2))
 (segment (start 96.925 92.7) (end 96.925 90.2) (width 0.4064) (layer F.Cu) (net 2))
 (segment (start 103.075 92.7) (end 96.925 92.7) (width 0.4064) (layer F.Cu) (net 2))
 (segment (start 105.125 95.175) (end 105.125 92.6) (width 0.4064) (layer F.Cu) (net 8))
 (segment (start 101.65 95.7) (end 104.6 95.7) (width 0.4064) (layer F.Cu) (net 8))
 (segment (start 104.6 95.7) (end 105.125 95.175) (width 0.4064) (layer F.Cu) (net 8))
 (segment (start 106.6 90.2) (end 105.125 90.2) (width 0.4064) (layer F.Cu) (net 9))
 (segment (start 107.2 90.8) (end 106.6 90.2) (width 0.4064) (layer F.Cu) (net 9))
 (segment (start 107.2 95.8) (end 107.2 90.8) (width 0.4064) (layer F.Cu) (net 9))
 (segment (start 100 98.5125) (end 104.4875 98.5125) (width 0.4064) (layer F.Cu) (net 9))
 (segment (start 104.4875 98.5125) (end 107.2 95.8) (width 0.4064) (layer F.Cu) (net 9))
 (segment (start 93.139088 108.5) (end 99.05 108.5) (width 0.4572) (layer B.Cu) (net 10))
 (segment (start 92.194544 107.555456) (end 93.139088 108.5) (width 0.4572) (layer B.Cu) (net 10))
 (segment (start 101 90.2) (end 100.95 90.25) (width 0.254) (layer F.Cu) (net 11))
 (segment (start 103.075 90.2) (end 101 90.2) (width 0.4064) (layer F.Cu) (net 11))
 (segment (start 86.475001 96.999998) (end 84.4 97) (width 0.4064) (layer F.Cu) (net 12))
 (segment (start 86.475001 103.000001) (end 84.4 103) (width 0.4064) (layer F.Cu) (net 12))
 (segment (start 113.625 103) (end 115.75 103) (width 0.4064) (layer F.Cu) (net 12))
 (segment (start 113.525 97) (end 115.75 97) (width 0.4064) (layer F.Cu) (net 12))
 (segment (start 90.073223 113.212311) (end 91.460912 114.6) (width 0.4572) (layer B.Cu) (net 12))
 (via (at 92.3 114.6) (size 1.016) (drill 0.508) (layers F.Cu B.Cu) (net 12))
 (segment (start 91.460912 114.6) (end 92.3 114.6) (width 0.4572) (layer B.Cu) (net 12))
 (segment (start 100 87.25) (end 100 85.9444) (width 0.4064) (layer F.Cu) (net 12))
 (segment (start 100 85.9444) (end 100 84.3) (width 0.4064) (layer F.Cu) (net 12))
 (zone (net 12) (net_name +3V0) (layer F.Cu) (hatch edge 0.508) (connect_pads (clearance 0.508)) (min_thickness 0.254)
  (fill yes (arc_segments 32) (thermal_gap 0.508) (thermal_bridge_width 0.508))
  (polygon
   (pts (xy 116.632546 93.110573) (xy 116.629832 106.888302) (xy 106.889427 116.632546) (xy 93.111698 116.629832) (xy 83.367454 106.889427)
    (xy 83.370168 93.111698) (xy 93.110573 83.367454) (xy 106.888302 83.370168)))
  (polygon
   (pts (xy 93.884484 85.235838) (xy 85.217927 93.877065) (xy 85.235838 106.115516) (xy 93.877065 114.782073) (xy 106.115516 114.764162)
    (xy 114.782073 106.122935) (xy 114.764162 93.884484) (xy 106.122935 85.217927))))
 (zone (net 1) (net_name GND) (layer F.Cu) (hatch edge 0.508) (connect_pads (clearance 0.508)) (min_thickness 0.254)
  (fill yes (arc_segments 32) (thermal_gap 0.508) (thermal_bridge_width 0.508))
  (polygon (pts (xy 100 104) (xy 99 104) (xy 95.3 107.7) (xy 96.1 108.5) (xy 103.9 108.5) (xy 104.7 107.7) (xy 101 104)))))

